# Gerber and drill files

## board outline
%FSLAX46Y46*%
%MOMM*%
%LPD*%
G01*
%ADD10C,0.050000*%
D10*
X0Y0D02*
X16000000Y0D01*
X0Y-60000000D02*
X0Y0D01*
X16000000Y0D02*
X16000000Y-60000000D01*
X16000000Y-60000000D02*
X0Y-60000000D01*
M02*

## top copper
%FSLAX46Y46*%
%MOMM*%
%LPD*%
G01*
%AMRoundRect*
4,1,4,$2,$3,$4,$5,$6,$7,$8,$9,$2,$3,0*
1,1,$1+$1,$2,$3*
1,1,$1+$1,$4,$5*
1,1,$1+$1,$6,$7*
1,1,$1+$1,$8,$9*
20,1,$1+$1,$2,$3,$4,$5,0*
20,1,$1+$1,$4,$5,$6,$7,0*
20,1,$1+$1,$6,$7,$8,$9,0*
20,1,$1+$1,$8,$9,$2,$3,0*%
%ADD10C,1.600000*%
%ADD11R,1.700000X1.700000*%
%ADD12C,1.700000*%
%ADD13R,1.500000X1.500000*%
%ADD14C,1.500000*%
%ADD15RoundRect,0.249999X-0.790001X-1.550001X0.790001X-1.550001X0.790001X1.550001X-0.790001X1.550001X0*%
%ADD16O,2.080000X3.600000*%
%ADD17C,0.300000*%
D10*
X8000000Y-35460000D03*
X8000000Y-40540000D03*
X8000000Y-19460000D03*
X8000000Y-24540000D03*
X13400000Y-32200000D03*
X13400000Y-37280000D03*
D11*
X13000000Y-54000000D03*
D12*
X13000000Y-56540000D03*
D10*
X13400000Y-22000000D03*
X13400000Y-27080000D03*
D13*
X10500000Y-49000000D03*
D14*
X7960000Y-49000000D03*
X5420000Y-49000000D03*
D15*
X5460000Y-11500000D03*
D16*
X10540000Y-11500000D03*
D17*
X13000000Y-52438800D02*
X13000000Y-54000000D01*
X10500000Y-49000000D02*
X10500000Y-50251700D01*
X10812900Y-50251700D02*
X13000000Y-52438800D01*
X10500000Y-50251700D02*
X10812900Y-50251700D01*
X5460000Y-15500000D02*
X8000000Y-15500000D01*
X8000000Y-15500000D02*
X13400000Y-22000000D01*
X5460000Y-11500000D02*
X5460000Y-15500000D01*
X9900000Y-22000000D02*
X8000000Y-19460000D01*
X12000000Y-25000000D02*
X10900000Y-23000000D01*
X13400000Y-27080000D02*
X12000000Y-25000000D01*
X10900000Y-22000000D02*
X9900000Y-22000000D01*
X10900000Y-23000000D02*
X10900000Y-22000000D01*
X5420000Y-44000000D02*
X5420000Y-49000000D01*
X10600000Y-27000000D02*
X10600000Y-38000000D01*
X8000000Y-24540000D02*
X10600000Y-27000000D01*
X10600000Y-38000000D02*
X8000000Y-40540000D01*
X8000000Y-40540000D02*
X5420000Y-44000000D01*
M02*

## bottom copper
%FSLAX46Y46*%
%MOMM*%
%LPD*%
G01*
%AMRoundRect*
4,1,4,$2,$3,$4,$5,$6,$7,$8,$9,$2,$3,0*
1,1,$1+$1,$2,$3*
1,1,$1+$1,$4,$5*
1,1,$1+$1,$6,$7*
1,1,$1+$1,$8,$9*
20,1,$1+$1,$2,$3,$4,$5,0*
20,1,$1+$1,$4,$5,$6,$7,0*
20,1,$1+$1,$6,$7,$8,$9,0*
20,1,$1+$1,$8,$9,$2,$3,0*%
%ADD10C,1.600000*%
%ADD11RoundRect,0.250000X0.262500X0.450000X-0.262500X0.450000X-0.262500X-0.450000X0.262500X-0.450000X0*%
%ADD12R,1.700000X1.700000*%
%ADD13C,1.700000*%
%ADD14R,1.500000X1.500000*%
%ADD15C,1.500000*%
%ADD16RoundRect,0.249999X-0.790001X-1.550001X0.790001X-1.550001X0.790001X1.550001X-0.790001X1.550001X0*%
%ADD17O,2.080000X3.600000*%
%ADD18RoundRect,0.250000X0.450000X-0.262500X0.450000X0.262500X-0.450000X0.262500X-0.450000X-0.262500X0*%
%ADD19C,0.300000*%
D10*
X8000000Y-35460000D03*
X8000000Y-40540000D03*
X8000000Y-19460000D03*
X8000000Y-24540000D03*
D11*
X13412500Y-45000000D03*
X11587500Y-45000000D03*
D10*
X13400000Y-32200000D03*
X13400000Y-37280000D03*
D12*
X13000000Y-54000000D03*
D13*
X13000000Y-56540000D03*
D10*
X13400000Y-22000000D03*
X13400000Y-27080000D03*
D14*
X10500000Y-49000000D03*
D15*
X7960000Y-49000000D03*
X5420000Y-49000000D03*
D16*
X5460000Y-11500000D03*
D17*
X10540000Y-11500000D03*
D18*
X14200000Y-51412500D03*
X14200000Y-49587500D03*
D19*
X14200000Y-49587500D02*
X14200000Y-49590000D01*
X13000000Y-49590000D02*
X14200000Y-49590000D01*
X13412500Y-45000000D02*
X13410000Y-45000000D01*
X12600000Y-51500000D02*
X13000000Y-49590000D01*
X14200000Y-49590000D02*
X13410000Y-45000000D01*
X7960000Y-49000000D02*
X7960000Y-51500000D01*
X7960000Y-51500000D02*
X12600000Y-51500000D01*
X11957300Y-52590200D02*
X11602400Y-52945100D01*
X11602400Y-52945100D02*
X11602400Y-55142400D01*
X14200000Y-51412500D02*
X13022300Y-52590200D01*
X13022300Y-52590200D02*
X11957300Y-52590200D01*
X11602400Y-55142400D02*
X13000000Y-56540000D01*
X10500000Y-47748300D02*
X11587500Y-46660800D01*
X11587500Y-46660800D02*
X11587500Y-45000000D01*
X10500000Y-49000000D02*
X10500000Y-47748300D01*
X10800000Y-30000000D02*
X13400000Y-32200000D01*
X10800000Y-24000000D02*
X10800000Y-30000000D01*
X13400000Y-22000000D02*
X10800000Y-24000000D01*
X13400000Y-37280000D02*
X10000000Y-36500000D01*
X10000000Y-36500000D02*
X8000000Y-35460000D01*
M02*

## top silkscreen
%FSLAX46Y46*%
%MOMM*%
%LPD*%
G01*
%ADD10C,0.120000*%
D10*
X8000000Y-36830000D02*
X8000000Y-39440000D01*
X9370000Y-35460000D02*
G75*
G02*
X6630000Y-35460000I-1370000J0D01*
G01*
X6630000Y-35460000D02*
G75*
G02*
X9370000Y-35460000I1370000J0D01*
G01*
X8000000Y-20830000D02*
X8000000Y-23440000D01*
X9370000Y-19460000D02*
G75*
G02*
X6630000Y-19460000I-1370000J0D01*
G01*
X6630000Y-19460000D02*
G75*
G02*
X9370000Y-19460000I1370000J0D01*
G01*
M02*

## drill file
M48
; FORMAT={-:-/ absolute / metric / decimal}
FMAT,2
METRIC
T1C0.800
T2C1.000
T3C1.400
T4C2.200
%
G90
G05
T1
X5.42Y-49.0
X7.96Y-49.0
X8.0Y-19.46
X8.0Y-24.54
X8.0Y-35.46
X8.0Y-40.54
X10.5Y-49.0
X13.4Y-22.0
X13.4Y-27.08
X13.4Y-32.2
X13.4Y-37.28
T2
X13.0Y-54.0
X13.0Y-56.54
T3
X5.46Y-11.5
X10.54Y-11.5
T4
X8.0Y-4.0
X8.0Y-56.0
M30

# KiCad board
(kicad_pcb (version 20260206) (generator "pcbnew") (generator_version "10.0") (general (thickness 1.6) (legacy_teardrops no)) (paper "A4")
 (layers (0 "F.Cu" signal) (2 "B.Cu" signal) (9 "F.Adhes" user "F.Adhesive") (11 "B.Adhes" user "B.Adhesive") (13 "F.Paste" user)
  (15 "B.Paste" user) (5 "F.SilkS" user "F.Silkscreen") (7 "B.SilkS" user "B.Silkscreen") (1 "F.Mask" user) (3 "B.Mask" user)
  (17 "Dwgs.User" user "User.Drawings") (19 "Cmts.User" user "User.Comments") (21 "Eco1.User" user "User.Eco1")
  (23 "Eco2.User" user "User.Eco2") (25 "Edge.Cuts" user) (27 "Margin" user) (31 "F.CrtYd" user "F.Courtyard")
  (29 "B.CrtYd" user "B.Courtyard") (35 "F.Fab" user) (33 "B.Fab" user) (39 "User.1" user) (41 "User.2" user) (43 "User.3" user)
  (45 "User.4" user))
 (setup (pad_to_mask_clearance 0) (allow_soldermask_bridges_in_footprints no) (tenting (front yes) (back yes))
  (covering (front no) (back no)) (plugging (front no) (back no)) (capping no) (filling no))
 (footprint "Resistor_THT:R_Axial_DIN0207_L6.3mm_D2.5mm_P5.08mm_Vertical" (layer "F.Cu") (at 8 35.46 -90)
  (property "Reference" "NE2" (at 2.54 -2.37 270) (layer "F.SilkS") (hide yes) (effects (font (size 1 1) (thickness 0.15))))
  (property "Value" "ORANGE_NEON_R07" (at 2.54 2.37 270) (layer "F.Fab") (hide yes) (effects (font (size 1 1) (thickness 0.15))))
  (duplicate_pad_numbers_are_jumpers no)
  (fp_line (start 1.37 0) (end 3.98 0) (stroke (width 0.12) (type solid)) (layer "F.SilkS"))
  (fp_circle (center 0 0) (end 1.37 0) (stroke (width 0.12) (type solid)) (fill no) (layer "F.SilkS"))
  (pad "1" thru_hole circle (at 0 0 270) (size 1.6 1.6) (drill 0.8) (layers "*.Cu" "*.Mask") (remove_unused_layers no) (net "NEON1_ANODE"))
  (pad "2" thru_hole circle (at 5.08 0 270) (size 1.6 1.6) (drill 0.8) (layers "*.Cu" "*.Mask") (remove_unused_layers no)
   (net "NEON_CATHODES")))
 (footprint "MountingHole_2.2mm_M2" (layer "F.Cu") (at 8 4)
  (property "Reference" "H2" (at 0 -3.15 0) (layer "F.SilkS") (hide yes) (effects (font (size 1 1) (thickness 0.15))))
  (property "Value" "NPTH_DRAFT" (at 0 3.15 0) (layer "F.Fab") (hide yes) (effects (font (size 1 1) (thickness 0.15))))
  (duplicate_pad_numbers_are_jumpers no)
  (pad "" np_thru_hole circle (at 0 0) (size 2.2 2.2) (drill 2.2) (layers "*.Cu" "*.Mask")))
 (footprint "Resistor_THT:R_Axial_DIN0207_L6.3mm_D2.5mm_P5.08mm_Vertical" (layer "F.Cu") (at 8 19.46 -90)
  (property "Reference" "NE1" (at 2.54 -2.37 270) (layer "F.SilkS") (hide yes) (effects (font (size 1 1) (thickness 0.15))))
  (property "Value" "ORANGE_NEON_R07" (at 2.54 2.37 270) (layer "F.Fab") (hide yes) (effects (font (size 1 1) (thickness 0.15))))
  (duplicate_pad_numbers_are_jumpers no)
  (fp_line (start 1.37 0) (end 3.98 0) (stroke (width 0.12) (type solid)) (layer "F.SilkS"))
  (fp_circle (center 0 0) (end 1.37 0) (stroke (width 0.12) (type solid)) (fill no) (layer "F.SilkS"))
  (pad "1" thru_hole circle (at 0 0 270) (size 1.6 1.6) (drill 0.8) (layers "*.Cu" "*.Mask") (remove_unused_layers no) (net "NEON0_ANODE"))
  (pad "2" thru_hole circle (at 5.08 0 270) (size 1.6 1.6) (drill 0.8) (layers "*.Cu" "*.Mask") (remove_unused_layers no)
   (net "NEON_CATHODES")))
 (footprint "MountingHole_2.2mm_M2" (layer "F.Cu") (at 8 56)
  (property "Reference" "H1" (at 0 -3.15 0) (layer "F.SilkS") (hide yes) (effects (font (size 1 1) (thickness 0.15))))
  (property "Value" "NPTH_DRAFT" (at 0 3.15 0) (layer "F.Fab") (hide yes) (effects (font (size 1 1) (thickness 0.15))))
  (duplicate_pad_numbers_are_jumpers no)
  (pad "" np_thru_hole circle (at 0 0) (size 2.2 2.2) (drill 2.2) (layers "*.Cu" "*.Mask")))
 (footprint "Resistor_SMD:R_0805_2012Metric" (layer "B.Cu") (at 12.5 45 180)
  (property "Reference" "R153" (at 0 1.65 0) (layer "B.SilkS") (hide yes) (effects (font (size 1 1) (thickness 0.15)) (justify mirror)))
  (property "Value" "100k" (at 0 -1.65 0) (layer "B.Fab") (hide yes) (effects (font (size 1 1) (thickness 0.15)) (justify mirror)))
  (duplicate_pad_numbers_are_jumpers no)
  (pad "1" smd roundrect (at -0.9125 0 180) (size 1.025 1.4) (layers "B.Cu" "B.Mask" "B.Paste") (roundrect_rratio 0.243902)
   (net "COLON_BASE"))
  (pad "2" smd roundrect (at 0.9125 0 180) (size 1.025 1.4) (layers "B.Cu" "B.Mask" "B.Paste") (roundrect_rratio 0.243902) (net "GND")))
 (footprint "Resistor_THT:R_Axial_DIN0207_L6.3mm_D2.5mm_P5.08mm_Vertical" (layer "B.Cu") (at 13.4 32.2 -90)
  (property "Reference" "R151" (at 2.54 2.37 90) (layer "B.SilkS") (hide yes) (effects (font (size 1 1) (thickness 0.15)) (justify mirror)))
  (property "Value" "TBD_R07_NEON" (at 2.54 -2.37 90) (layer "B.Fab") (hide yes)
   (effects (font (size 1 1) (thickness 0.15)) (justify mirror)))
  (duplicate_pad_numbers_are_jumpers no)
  (pad "1" thru_hole circle (at 0 0 270) (size 1.6 1.6) (drill 0.8) (layers "*.Cu" "*.Mask") (remove_unused_layers no) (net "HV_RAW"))
  (pad "2" thru_hole circle (at 5.08 0 270) (size 1.6 1.6) (drill 0.8) (layers "*.Cu" "*.Mask") (remove_unused_layers no)
   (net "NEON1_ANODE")))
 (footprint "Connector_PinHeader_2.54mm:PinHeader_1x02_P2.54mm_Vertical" (layer "B.Cu") (at 13 54 180)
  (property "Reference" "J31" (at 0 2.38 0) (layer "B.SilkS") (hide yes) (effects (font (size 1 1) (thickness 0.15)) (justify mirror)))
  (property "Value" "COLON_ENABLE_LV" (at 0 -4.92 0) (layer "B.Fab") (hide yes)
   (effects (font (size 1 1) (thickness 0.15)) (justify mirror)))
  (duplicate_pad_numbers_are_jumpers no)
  (pad "1" thru_hole rect (at 0 0 180) (size 1.7 1.7) (drill 1) (layers "*.Cu" "*.Mask") (remove_unused_layers no) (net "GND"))
  (pad "2" thru_hole circle (at 0 -2.54 180) (size 1.7 1.7) (drill 1) (layers "*.Cu" "*.Mask") (remove_unused_layers no)
   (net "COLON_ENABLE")))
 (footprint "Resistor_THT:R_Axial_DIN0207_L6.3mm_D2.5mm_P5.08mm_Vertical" (layer "B.Cu") (at 13.4 22 -90)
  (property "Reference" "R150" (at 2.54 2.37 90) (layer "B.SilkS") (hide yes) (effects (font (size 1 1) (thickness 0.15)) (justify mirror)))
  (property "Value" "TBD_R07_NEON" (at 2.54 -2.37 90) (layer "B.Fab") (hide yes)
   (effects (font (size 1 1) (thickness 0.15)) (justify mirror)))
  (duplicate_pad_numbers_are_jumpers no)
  (pad "1" thru_hole circle (at 0 0 270) (size 1.6 1.6) (drill 0.8) (layers "*.Cu" "*.Mask") (remove_unused_layers no) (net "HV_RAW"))
  (pad "2" thru_hole circle (at 5.08 0 270) (size 1.6 1.6) (drill 0.8) (layers "*.Cu" "*.Mask") (remove_unused_layers no)
   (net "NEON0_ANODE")))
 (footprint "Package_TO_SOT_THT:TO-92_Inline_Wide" (layer "B.Cu") (at 10.5 49 180)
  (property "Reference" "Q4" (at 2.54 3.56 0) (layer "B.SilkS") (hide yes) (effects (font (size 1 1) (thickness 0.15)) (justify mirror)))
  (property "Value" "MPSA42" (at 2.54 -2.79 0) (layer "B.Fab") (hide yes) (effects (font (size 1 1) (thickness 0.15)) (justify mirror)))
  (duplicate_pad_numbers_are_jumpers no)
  (pad "1" thru_hole rect (at 0 0 180) (size 1.5 1.5) (drill 0.8) (layers "*.Cu" "*.Mask") (remove_unused_layers no) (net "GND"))
  (pad "2" thru_hole circle (at 2.54 0 180) (size 1.5 1.5) (drill 0.8) (layers "*.Cu" "*.Mask") (remove_unused_layers no) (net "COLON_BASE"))
  (pad "3" thru_hole circle (at 5.08 0 180) (size 1.5 1.5) (drill 0.8) (layers "*.Cu" "*.Mask") (remove_unused_layers no)
   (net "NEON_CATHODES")))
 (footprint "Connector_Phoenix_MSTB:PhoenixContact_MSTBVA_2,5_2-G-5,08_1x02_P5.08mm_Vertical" (layer "B.Cu") (at 5.46 11.5)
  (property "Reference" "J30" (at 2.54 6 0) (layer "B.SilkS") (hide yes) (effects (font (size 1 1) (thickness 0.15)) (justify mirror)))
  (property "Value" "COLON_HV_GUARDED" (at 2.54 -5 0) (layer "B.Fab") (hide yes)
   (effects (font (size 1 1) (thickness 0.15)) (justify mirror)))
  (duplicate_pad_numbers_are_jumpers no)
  (pad "1" thru_hole roundrect (at 0 0) (size 2.08 3.6) (drill 1.4) (layers "*.Cu" "*.Mask") (remove_unused_layers no)
   (roundrect_rratio 0.120192) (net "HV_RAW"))
  (pad "2" thru_hole oval (at 5.08 0) (size 2.08 3.6) (drill 1.4) (layers "*.Cu" "*.Mask") (remove_unused_layers no)
   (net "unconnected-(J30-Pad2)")))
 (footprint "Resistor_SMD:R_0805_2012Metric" (layer "B.Cu") (at 14.2 50.5 90)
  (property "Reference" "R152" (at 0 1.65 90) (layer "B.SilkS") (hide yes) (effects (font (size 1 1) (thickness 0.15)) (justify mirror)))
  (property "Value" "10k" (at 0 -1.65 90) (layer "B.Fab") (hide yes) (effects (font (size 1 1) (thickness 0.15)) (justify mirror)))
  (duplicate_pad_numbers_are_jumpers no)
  (pad "1" smd roundrect (at -0.9125 0 90) (size 1.025 1.4) (layers "B.Cu" "B.Mask" "B.Paste") (roundrect_rratio 0.243902)
   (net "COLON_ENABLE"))
  (pad "2" smd roundrect (at 0.9125 0 90) (size 1.025 1.4) (layers "B.Cu" "B.Mask" "B.Paste") (roundrect_rratio 0.243902) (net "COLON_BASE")))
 (gr_line (start 0 0) (end 16 0) (stroke (width 0.05) (type default)) (layer "Edge.Cuts"))
 (gr_line (start 0 60) (end 0 0) (stroke (width 0.05) (type default)) (layer "Edge.Cuts"))
 (gr_line (start 16 0) (end 16 60) (stroke (width 0.05) (type default)) (layer "Edge.Cuts"))
 (gr_line (start 16 60) (end 0 60) (stroke (width 0.05) (type default)) (layer "Edge.Cuts"))
 (segment (start 14.2 49.5875) (end 14.2 49.59) (width 0.3) (layer "B.Cu") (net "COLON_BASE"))
 (segment (start 13 49.59) (end 14.2 49.59) (width 0.3) (layer "B.Cu") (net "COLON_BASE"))
 (segment (start 13.4125 45) (end 13.41 45) (width 0.3) (layer "B.Cu") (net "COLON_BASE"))
 (segment (start 12.6 51.5) (end 13 49.59) (width 0.3) (layer "B.Cu") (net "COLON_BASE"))
 (segment (start 14.2 49.59) (end 13.41 45) (width 0.3) (layer "B.Cu") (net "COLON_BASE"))
 (segment (start 7.96 49) (end 7.96 51.5) (width 0.3) (layer "B.Cu") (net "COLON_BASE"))
 (segment (start 7.96 51.5) (end 12.6 51.5) (width 0.3) (layer "B.Cu") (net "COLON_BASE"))
 (segment (start 11.9573 52.5902) (end 11.6024 52.9451) (width 0.3) (layer "B.Cu") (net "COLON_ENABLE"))
 (segment (start 11.6024 52.9451) (end 11.6024 55.1424) (width 0.3) (layer "B.Cu") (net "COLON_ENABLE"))
 (segment (start 14.2 51.4125) (end 13.0223 52.5902) (width 0.3) (layer "B.Cu") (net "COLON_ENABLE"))
 (segment (start 13.0223 52.5902) (end 11.9573 52.5902) (width 0.3) (layer "B.Cu") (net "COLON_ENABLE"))
 (segment (start 11.6024 55.1424) (end 13 56.54) (width 0.3) (layer "B.Cu") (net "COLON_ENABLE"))
 (segment (start 13 52.4388) (end 13 54) (width 0.3) (layer "F.Cu") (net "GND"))
 (segment (start 10.5 49) (end 10.5 50.2517) (width 0.3) (layer "F.Cu") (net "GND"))
 (segment (start 10.8129 50.2517) (end 13 52.4388) (width 0.3) (layer "F.Cu") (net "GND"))
 (segment (start 10.5 50.2517) (end 10.8129 50.2517) (width 0.3) (layer "F.Cu") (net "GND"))
 (segment (start 10.5 47.7483) (end 11.5875 46.6608) (width 0.3) (layer "B.Cu") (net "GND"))
 (segment (start 11.5875 46.6608) (end 11.5875 45) (width 0.3) (layer "B.Cu") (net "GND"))
 (segment (start 10.5 49) (end 10.5 47.7483) (width 0.3) (layer "B.Cu") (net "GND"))
 (segment (start 5.46 15.5) (end 8 15.5) (width 0.3) (layer "F.Cu") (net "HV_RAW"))
 (segment (start 8 15.5) (end 13.4 22) (width 0.3) (layer "F.Cu") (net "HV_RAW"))
 (segment (start 5.46 11.5) (end 5.46 15.5) (width 0.3) (layer "F.Cu") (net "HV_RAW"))
 (segment (start 10.8 30) (end 13.4 32.2) (width 0.3) (layer "B.Cu") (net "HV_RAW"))
 (segment (start 10.8 24) (end 10.8 30) (width 0.3) (layer "B.Cu") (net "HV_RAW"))
 (segment (start 13.4 22) (end 10.8 24) (width 0.3) (layer "B.Cu") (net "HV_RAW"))
 (segment (start 9.9 22) (end 8 19.46) (width 0.3) (layer "F.Cu") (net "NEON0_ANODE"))
 (segment (start 12 25) (end 10.9 23) (width 0.3) (layer "F.Cu") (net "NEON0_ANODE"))
 (segment (start 13.4 27.08) (end 12 25) (width 0.3) (layer "F.Cu") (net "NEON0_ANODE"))
 (segment (start 10.9 22) (end 9.9 22) (width 0.3) (layer "F.Cu") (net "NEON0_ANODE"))
 (segment (start 10.9 23) (end 10.9 22) (width 0.3) (layer "F.Cu") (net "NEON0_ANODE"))
 (segment (start 13.4 37.28) (end 10 36.5) (width 0.3) (layer "B.Cu") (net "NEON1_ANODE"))
 (segment (start 10 36.5) (end 8 35.46) (width 0.3) (layer "B.Cu") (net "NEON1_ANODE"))
 (segment (start 5.42 44) (end 5.42 49) (width 0.3) (layer "F.Cu") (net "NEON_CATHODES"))
 (segment (start 10.6 27) (end 10.6 38) (width 0.3) (layer "F.Cu") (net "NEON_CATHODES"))
 (segment (start 8 24.54) (end 10.6 27) (width 0.3) (layer "F.Cu") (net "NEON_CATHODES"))
 (segment (start 10.6 38) (end 8 40.54) (width 0.3) (layer "F.Cu") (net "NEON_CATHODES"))
 (segment (start 8 40.54) (end 5.42 44) (width 0.3) (layer "F.Cu") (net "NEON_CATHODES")))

